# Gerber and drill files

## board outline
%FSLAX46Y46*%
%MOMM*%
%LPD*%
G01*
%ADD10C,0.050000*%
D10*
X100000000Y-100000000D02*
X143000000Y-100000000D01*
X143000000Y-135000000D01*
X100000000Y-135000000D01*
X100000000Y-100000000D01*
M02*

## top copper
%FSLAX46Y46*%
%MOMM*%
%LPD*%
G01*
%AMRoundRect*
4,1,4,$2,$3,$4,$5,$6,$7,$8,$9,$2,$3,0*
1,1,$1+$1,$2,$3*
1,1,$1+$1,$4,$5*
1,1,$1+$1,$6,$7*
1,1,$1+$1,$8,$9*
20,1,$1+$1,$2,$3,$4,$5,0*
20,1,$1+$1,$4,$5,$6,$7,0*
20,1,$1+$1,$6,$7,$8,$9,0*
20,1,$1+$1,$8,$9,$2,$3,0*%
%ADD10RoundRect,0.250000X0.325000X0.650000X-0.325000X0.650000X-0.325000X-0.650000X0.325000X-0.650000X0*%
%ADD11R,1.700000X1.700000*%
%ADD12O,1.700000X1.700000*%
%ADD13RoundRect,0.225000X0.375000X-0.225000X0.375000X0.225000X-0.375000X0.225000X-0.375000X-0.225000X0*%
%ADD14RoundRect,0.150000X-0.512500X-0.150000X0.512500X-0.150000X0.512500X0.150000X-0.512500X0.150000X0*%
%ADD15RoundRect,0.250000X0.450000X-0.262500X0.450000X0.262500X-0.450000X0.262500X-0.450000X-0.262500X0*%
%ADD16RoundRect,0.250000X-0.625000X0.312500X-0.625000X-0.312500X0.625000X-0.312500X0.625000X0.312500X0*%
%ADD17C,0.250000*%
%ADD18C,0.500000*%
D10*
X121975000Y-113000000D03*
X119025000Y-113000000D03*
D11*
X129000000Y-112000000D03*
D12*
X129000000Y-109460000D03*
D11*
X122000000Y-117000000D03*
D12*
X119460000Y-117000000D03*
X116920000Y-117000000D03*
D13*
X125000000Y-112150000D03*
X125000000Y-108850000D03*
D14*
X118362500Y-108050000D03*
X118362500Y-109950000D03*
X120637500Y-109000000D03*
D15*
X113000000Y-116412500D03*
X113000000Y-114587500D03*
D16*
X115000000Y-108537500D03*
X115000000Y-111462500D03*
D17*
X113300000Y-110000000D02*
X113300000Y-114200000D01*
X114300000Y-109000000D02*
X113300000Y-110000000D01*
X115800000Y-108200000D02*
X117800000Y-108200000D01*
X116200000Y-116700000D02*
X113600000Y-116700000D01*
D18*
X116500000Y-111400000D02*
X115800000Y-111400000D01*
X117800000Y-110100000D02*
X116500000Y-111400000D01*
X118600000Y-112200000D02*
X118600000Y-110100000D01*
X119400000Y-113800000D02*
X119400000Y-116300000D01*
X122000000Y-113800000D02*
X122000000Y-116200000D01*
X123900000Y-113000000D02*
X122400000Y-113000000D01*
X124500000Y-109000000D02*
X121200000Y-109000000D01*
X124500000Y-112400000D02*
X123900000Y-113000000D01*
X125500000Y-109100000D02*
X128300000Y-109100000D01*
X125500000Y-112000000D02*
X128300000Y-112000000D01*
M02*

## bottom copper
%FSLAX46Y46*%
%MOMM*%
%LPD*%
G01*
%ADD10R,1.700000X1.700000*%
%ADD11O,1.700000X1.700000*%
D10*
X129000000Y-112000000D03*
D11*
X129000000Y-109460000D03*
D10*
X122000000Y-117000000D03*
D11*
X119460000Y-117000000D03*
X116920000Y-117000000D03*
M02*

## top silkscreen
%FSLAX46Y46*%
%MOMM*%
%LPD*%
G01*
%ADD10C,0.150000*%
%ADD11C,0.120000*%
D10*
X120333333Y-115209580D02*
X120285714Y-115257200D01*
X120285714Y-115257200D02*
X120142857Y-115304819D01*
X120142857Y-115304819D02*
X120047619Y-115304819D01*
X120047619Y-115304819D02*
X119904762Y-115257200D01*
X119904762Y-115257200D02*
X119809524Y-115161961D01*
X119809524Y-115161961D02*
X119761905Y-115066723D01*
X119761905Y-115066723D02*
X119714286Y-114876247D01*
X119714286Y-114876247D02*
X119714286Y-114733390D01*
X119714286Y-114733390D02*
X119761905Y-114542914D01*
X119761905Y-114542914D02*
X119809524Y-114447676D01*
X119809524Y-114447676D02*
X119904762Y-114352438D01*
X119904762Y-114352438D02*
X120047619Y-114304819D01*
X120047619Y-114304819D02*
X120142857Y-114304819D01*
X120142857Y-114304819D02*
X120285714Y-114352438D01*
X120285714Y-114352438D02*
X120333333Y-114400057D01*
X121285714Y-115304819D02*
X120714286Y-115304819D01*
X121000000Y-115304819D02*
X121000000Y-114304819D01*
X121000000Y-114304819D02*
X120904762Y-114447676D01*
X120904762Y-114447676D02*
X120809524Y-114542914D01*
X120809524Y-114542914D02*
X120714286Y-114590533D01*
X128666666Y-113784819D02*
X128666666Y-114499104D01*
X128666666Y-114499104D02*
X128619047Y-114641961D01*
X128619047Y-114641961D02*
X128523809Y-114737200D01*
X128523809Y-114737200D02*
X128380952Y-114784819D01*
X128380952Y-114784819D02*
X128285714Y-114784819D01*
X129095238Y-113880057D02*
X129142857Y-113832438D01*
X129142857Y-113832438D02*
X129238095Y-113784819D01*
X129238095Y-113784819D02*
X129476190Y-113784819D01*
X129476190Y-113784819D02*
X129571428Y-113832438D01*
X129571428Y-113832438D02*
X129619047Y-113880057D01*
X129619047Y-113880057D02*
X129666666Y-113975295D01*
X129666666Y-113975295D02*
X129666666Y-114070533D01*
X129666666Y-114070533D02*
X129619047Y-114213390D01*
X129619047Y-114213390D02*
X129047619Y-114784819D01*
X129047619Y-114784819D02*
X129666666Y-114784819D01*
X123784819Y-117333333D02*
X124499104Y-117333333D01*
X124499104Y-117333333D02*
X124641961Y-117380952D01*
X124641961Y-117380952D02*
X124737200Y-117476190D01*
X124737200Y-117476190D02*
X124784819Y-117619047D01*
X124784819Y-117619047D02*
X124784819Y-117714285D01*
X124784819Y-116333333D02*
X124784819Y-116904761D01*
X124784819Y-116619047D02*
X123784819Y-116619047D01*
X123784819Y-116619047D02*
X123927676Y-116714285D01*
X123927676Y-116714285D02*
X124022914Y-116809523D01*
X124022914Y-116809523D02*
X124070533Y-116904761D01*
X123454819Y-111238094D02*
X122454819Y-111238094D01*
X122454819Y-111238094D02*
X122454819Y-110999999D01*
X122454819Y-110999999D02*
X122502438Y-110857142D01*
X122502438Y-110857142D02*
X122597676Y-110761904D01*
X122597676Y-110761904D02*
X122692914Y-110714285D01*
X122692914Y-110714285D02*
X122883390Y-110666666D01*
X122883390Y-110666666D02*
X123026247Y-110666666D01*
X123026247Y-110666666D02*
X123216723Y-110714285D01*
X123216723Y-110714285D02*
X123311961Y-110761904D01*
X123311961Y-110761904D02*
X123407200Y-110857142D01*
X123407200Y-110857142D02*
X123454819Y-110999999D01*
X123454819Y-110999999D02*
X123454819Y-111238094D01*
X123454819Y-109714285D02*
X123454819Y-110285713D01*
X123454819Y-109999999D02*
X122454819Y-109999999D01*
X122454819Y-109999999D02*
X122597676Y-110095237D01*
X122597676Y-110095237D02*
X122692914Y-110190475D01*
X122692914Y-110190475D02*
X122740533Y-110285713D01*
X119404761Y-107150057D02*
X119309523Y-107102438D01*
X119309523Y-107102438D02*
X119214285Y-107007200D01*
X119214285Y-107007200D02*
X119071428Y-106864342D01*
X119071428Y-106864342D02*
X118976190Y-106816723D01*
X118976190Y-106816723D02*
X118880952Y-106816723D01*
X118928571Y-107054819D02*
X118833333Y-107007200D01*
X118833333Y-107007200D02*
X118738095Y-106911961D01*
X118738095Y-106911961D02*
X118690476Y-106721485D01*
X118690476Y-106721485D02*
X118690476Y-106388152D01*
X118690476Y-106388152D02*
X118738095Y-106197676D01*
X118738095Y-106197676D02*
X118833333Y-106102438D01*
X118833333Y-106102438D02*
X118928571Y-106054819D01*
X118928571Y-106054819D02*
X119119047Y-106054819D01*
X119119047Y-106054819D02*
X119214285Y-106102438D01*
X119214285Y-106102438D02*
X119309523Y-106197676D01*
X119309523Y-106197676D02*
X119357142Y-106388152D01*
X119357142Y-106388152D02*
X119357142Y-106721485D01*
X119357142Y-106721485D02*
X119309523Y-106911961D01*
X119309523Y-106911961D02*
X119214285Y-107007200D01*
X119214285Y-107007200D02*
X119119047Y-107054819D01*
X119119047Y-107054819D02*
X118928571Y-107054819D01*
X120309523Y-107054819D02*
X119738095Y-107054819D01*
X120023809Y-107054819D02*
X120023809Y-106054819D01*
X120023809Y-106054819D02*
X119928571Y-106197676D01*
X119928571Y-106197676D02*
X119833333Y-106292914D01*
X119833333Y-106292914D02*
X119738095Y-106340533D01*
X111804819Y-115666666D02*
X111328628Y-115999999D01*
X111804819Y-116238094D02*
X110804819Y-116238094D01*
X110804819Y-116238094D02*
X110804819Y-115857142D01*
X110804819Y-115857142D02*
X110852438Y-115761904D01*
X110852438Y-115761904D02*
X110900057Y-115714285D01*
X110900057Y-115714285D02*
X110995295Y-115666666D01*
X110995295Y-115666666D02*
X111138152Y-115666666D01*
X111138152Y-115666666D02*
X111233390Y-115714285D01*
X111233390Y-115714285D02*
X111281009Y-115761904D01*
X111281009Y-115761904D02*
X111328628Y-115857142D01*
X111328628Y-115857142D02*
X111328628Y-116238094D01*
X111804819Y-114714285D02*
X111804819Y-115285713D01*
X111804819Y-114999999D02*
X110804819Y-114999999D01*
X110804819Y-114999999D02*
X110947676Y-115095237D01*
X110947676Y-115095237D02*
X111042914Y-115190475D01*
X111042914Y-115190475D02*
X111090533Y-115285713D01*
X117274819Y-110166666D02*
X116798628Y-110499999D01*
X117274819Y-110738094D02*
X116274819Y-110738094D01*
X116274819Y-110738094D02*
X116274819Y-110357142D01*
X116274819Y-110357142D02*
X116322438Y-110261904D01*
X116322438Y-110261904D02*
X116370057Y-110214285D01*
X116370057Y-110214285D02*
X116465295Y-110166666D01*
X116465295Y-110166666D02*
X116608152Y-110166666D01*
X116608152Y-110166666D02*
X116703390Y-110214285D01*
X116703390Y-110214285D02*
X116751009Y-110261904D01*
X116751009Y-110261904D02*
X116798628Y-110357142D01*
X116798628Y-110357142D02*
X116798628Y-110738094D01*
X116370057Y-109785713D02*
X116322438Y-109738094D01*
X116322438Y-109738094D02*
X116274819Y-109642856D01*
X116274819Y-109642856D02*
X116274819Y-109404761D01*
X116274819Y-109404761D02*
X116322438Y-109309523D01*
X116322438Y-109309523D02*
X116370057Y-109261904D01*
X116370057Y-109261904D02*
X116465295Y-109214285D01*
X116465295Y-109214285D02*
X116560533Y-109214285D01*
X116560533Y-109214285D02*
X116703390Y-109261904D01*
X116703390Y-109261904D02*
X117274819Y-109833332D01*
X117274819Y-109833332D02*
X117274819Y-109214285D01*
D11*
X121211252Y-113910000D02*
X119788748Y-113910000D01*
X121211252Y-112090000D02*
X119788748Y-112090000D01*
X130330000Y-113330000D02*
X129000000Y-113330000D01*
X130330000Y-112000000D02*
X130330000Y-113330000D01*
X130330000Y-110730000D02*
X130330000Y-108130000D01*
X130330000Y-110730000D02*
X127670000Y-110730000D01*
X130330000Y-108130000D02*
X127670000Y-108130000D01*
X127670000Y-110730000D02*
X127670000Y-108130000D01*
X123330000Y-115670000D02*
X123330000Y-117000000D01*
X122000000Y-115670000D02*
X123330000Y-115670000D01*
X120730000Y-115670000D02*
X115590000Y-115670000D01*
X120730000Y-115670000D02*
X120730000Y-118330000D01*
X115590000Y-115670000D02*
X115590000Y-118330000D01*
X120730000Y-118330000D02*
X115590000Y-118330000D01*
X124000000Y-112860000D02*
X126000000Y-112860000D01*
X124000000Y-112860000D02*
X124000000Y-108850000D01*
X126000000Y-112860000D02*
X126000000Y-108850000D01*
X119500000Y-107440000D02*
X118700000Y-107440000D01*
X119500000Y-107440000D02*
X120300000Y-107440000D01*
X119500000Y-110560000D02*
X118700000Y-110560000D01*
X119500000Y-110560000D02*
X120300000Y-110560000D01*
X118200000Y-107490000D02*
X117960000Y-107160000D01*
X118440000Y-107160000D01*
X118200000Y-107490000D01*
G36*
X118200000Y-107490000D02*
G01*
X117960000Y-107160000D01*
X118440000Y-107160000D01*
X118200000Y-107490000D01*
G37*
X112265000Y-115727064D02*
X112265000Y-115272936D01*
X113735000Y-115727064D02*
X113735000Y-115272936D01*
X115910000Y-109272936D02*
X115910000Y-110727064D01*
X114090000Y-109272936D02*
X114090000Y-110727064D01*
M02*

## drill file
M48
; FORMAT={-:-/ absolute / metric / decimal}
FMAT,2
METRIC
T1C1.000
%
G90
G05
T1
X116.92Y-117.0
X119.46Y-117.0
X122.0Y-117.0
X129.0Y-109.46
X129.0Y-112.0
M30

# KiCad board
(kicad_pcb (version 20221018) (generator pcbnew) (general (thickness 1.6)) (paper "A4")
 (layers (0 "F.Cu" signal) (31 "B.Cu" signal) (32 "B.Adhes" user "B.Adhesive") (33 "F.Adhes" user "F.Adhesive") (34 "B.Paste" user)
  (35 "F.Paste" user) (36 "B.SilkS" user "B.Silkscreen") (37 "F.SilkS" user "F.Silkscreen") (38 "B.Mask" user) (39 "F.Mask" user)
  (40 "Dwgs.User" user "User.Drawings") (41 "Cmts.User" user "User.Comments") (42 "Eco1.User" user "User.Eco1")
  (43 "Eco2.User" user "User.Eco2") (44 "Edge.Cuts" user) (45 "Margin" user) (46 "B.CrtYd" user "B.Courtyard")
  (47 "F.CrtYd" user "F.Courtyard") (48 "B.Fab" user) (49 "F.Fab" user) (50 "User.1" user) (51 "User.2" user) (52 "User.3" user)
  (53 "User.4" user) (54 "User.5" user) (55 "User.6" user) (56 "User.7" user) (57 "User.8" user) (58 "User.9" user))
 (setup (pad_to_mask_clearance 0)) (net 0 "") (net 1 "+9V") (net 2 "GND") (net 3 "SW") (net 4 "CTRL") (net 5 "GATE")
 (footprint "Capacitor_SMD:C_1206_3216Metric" (layer "F.Cu") (at 120.5 113 180)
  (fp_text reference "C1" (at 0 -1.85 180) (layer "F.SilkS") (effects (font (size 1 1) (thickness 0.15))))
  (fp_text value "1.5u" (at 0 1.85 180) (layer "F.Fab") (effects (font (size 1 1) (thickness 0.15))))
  (fp_line (start -0.711252 -0.91) (end 0.711252 -0.91) (stroke (width 0.12) (type solid)) (layer "F.SilkS"))
  (fp_line (start -0.711252 0.91) (end 0.711252 0.91) (stroke (width 0.12) (type solid)) (layer "F.SilkS"))
  (pad "1" smd roundrect (at -1.475 0 180) (size 1.15 1.8) (layers "F.Cu" "F.Paste" "F.Mask") (roundrect_rratio 0.217391) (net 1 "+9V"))
  (pad "2" smd roundrect (at 1.475 0 180) (size 1.15 1.8) (layers "F.Cu" "F.Paste" "F.Mask") (roundrect_rratio 0.217391) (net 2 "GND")))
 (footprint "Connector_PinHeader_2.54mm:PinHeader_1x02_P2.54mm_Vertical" (layer "F.Cu") (at 129 112 180)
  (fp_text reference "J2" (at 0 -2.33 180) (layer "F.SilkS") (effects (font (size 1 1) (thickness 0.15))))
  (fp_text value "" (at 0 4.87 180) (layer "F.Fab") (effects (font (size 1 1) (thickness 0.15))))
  (fp_line (start -1.33 -1.33) (end 0 -1.33) (stroke (width 0.12) (type solid)) (layer "F.SilkS"))
  (fp_line (start -1.33 0) (end -1.33 -1.33) (stroke (width 0.12) (type solid)) (layer "F.SilkS"))
  (fp_line (start -1.33 1.27) (end -1.33 3.87) (stroke (width 0.12) (type solid)) (layer "F.SilkS"))
  (fp_line (start -1.33 1.27) (end 1.33 1.27) (stroke (width 0.12) (type solid)) (layer "F.SilkS"))
  (fp_line (start -1.33 3.87) (end 1.33 3.87) (stroke (width 0.12) (type solid)) (layer "F.SilkS"))
  (fp_line (start 1.33 1.27) (end 1.33 3.87) (stroke (width 0.12) (type solid)) (layer "F.SilkS"))
  (pad "1" thru_hole rect (at 0 0 180) (size 1.7 1.7) (drill 1) (layers "*.Cu" "*.Mask") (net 1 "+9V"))
  (pad "2" thru_hole oval (at 0 2.54 180) (size 1.7 1.7) (drill 1) (layers "*.Cu" "*.Mask") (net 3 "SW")))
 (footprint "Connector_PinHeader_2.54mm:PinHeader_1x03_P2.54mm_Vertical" (layer "F.Cu") (at 122 117 -90)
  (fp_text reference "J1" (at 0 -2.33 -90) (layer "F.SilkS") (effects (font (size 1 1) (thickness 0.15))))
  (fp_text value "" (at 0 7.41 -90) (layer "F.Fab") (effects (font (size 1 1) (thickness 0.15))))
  (fp_line (start -1.33 -1.33) (end 0 -1.33) (stroke (width 0.12) (type solid)) (layer "F.SilkS"))
  (fp_line (start -1.33 0) (end -1.33 -1.33) (stroke (width 0.12) (type solid)) (layer "F.SilkS"))
  (fp_line (start -1.33 1.27) (end -1.33 6.41) (stroke (width 0.12) (type solid)) (layer "F.SilkS"))
  (fp_line (start -1.33 1.27) (end 1.33 1.27) (stroke (width 0.12) (type solid)) (layer "F.SilkS"))
  (fp_line (start -1.33 6.41) (end 1.33 6.41) (stroke (width 0.12) (type solid)) (layer "F.SilkS"))
  (fp_line (start 1.33 1.27) (end 1.33 6.41) (stroke (width 0.12) (type solid)) (layer "F.SilkS"))
  (pad "1" thru_hole rect (at 0 0 270) (size 1.7 1.7) (drill 1) (layers "*.Cu" "*.Mask") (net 1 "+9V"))
  (pad "2" thru_hole oval (at 0 2.54 270) (size 1.7 1.7) (drill 1) (layers "*.Cu" "*.Mask") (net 2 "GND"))
  (pad "3" thru_hole oval (at 0 5.08 270) (size 1.7 1.7) (drill 1) (layers "*.Cu" "*.Mask") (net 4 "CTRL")))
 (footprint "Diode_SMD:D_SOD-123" (layer "F.Cu") (at 125 110.5 90)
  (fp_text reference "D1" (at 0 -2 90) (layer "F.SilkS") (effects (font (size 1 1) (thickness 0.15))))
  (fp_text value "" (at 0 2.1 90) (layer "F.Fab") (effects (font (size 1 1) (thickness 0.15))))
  (fp_line (start -2.36 -1) (end -2.36 1) (stroke (width 0.12) (type solid)) (layer "F.SilkS"))
  (fp_line (start -2.36 -1) (end 1.65 -1) (stroke (width 0.12) (type solid)) (layer "F.SilkS"))
  (fp_line (start -2.36 1) (end 1.65 1) (stroke (width 0.12) (type solid)) (layer "F.SilkS"))
  (pad "1" smd roundrect (at -1.65 0 90) (size 0.9 1.2) (layers "F.Cu" "F.Paste" "F.Mask") (roundrect_rratio 0.25) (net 1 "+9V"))
  (pad "2" smd roundrect (at 1.65 0 90) (size 0.9 1.2) (layers "F.Cu" "F.Paste" "F.Mask") (roundrect_rratio 0.25) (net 3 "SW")))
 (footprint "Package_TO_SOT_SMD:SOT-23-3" (layer "F.Cu") (at 119.5 109)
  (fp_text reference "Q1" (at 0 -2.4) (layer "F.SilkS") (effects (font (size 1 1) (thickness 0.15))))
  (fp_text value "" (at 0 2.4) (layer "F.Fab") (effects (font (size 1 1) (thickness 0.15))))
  (fp_line (start 0 -1.56) (end -0.8 -1.56) (stroke (width 0.12) (type solid)) (layer "F.SilkS"))
  (fp_line (start 0 -1.56) (end 0.8 -1.56) (stroke (width 0.12) (type solid)) (layer "F.SilkS"))
  (fp_line (start 0 1.56) (end -0.8 1.56) (stroke (width 0.12) (type solid)) (layer "F.SilkS"))
  (fp_line (start 0 1.56) (end 0.8 1.56) (stroke (width 0.12) (type solid)) (layer "F.SilkS"))
  (fp_poly
   (pts (xy -1.3 -1.51) (xy -1.54 -1.84) (xy -1.06 -1.84) (xy -1.3 -1.51)) (stroke (width 0.12) (type solid)) (fill solid) (layer "F.SilkS"))
  (pad "1" smd roundrect (at -1.1375 -0.95) (size 1.325 0.6) (layers "F.Cu" "F.Paste" "F.Mask") (roundrect_rratio 0.25) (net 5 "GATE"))
  (pad "2" smd roundrect (at -1.1375 0.95) (size 1.325 0.6) (layers "F.Cu" "F.Paste" "F.Mask") (roundrect_rratio 0.25) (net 2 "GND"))
  (pad "3" smd roundrect (at 1.1375 0) (size 1.325 0.6) (layers "F.Cu" "F.Paste" "F.Mask") (roundrect_rratio 0.25) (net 3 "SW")))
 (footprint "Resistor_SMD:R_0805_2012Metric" (layer "F.Cu") (at 113 115.5 90)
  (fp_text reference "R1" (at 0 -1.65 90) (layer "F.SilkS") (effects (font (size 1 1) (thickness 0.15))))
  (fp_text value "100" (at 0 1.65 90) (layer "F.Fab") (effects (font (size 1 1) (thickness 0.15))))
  (fp_line (start -0.227064 -0.735) (end 0.227064 -0.735) (stroke (width 0.12) (type solid)) (layer "F.SilkS"))
  (fp_line (start -0.227064 0.735) (end 0.227064 0.735) (stroke (width 0.12) (type solid)) (layer "F.SilkS"))
  (pad "1" smd roundrect (at -0.9125 0 90) (size 1.025 1.4) (layers "F.Cu" "F.Paste" "F.Mask") (roundrect_rratio 0.243902) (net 4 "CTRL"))
  (pad "2" smd roundrect (at 0.9125 0 90) (size 1.025 1.4) (layers "F.Cu" "F.Paste" "F.Mask") (roundrect_rratio 0.243902) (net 5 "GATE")))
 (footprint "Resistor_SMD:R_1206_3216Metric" (layer "F.Cu") (at 115 110 -90)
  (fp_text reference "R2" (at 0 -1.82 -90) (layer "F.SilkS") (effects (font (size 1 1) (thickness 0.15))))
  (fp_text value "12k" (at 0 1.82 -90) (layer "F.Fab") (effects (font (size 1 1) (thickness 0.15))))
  (fp_line (start -0.727064 -0.91) (end 0.727064 -0.91) (stroke (width 0.12) (type solid)) (layer "F.SilkS"))
  (fp_line (start -0.727064 0.91) (end 0.727064 0.91) (stroke (width 0.12) (type solid)) (layer "F.SilkS"))
  (pad "1" smd roundrect (at -1.4625 0 270) (size 1.125 1.75) (layers "F.Cu" "F.Paste" "F.Mask") (roundrect_rratio 0.222222) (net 5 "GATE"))
  (pad "2" smd roundrect (at 1.4625 0 270) (size 1.125 1.75) (layers "F.Cu" "F.Paste" "F.Mask") (roundrect_rratio 0.222222) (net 2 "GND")))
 (gr_rect (start 100 100) (end 143 135) (stroke (width 0.05) (type default)) (fill none) (layer "Edge.Cuts"))
 (segment (start 113.3 110) (end 113.3 114.2) (width 0.25) (layer "F.Cu") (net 5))
 (segment (start 114.3 109) (end 113.3 110) (width 0.25) (layer "F.Cu") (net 5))
 (segment (start 115.8 108.2) (end 117.8 108.2) (width 0.25) (layer "F.Cu") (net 5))
 (segment (start 116.2 116.7) (end 113.6 116.7) (width 0.25) (layer "F.Cu") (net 4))
 (segment (start 116.5 111.4) (end 115.8 111.4) (width 0.5) (layer "F.Cu") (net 2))
 (segment (start 117.8 110.1) (end 116.5 111.4) (width 0.5) (layer "F.Cu") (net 2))
 (segment (start 118.6 112.2) (end 118.6 110.1) (width 0.5) (layer "F.Cu") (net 2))
 (segment (start 119.4 113.8) (end 119.4 116.3) (width 0.5) (layer "F.Cu") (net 2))
 (segment (start 122 113.8) (end 122 116.2) (width 0.5) (layer "F.Cu") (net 1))
 (segment (start 123.9 113) (end 122.4 113) (width 0.5) (layer "F.Cu") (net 1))
 (segment (start 124.5 109) (end 121.2 109) (width 0.5) (layer "F.Cu") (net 3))
 (segment (start 124.5 112.4) (end 123.9 113) (width 0.5) (layer "F.Cu") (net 1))
 (segment (start 125.5 109.1) (end 128.3 109.1) (width 0.5) (layer "F.Cu") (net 3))
 (segment (start 125.5 112) (end 128.3 112) (width 0.5) (layer "F.Cu") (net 1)))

